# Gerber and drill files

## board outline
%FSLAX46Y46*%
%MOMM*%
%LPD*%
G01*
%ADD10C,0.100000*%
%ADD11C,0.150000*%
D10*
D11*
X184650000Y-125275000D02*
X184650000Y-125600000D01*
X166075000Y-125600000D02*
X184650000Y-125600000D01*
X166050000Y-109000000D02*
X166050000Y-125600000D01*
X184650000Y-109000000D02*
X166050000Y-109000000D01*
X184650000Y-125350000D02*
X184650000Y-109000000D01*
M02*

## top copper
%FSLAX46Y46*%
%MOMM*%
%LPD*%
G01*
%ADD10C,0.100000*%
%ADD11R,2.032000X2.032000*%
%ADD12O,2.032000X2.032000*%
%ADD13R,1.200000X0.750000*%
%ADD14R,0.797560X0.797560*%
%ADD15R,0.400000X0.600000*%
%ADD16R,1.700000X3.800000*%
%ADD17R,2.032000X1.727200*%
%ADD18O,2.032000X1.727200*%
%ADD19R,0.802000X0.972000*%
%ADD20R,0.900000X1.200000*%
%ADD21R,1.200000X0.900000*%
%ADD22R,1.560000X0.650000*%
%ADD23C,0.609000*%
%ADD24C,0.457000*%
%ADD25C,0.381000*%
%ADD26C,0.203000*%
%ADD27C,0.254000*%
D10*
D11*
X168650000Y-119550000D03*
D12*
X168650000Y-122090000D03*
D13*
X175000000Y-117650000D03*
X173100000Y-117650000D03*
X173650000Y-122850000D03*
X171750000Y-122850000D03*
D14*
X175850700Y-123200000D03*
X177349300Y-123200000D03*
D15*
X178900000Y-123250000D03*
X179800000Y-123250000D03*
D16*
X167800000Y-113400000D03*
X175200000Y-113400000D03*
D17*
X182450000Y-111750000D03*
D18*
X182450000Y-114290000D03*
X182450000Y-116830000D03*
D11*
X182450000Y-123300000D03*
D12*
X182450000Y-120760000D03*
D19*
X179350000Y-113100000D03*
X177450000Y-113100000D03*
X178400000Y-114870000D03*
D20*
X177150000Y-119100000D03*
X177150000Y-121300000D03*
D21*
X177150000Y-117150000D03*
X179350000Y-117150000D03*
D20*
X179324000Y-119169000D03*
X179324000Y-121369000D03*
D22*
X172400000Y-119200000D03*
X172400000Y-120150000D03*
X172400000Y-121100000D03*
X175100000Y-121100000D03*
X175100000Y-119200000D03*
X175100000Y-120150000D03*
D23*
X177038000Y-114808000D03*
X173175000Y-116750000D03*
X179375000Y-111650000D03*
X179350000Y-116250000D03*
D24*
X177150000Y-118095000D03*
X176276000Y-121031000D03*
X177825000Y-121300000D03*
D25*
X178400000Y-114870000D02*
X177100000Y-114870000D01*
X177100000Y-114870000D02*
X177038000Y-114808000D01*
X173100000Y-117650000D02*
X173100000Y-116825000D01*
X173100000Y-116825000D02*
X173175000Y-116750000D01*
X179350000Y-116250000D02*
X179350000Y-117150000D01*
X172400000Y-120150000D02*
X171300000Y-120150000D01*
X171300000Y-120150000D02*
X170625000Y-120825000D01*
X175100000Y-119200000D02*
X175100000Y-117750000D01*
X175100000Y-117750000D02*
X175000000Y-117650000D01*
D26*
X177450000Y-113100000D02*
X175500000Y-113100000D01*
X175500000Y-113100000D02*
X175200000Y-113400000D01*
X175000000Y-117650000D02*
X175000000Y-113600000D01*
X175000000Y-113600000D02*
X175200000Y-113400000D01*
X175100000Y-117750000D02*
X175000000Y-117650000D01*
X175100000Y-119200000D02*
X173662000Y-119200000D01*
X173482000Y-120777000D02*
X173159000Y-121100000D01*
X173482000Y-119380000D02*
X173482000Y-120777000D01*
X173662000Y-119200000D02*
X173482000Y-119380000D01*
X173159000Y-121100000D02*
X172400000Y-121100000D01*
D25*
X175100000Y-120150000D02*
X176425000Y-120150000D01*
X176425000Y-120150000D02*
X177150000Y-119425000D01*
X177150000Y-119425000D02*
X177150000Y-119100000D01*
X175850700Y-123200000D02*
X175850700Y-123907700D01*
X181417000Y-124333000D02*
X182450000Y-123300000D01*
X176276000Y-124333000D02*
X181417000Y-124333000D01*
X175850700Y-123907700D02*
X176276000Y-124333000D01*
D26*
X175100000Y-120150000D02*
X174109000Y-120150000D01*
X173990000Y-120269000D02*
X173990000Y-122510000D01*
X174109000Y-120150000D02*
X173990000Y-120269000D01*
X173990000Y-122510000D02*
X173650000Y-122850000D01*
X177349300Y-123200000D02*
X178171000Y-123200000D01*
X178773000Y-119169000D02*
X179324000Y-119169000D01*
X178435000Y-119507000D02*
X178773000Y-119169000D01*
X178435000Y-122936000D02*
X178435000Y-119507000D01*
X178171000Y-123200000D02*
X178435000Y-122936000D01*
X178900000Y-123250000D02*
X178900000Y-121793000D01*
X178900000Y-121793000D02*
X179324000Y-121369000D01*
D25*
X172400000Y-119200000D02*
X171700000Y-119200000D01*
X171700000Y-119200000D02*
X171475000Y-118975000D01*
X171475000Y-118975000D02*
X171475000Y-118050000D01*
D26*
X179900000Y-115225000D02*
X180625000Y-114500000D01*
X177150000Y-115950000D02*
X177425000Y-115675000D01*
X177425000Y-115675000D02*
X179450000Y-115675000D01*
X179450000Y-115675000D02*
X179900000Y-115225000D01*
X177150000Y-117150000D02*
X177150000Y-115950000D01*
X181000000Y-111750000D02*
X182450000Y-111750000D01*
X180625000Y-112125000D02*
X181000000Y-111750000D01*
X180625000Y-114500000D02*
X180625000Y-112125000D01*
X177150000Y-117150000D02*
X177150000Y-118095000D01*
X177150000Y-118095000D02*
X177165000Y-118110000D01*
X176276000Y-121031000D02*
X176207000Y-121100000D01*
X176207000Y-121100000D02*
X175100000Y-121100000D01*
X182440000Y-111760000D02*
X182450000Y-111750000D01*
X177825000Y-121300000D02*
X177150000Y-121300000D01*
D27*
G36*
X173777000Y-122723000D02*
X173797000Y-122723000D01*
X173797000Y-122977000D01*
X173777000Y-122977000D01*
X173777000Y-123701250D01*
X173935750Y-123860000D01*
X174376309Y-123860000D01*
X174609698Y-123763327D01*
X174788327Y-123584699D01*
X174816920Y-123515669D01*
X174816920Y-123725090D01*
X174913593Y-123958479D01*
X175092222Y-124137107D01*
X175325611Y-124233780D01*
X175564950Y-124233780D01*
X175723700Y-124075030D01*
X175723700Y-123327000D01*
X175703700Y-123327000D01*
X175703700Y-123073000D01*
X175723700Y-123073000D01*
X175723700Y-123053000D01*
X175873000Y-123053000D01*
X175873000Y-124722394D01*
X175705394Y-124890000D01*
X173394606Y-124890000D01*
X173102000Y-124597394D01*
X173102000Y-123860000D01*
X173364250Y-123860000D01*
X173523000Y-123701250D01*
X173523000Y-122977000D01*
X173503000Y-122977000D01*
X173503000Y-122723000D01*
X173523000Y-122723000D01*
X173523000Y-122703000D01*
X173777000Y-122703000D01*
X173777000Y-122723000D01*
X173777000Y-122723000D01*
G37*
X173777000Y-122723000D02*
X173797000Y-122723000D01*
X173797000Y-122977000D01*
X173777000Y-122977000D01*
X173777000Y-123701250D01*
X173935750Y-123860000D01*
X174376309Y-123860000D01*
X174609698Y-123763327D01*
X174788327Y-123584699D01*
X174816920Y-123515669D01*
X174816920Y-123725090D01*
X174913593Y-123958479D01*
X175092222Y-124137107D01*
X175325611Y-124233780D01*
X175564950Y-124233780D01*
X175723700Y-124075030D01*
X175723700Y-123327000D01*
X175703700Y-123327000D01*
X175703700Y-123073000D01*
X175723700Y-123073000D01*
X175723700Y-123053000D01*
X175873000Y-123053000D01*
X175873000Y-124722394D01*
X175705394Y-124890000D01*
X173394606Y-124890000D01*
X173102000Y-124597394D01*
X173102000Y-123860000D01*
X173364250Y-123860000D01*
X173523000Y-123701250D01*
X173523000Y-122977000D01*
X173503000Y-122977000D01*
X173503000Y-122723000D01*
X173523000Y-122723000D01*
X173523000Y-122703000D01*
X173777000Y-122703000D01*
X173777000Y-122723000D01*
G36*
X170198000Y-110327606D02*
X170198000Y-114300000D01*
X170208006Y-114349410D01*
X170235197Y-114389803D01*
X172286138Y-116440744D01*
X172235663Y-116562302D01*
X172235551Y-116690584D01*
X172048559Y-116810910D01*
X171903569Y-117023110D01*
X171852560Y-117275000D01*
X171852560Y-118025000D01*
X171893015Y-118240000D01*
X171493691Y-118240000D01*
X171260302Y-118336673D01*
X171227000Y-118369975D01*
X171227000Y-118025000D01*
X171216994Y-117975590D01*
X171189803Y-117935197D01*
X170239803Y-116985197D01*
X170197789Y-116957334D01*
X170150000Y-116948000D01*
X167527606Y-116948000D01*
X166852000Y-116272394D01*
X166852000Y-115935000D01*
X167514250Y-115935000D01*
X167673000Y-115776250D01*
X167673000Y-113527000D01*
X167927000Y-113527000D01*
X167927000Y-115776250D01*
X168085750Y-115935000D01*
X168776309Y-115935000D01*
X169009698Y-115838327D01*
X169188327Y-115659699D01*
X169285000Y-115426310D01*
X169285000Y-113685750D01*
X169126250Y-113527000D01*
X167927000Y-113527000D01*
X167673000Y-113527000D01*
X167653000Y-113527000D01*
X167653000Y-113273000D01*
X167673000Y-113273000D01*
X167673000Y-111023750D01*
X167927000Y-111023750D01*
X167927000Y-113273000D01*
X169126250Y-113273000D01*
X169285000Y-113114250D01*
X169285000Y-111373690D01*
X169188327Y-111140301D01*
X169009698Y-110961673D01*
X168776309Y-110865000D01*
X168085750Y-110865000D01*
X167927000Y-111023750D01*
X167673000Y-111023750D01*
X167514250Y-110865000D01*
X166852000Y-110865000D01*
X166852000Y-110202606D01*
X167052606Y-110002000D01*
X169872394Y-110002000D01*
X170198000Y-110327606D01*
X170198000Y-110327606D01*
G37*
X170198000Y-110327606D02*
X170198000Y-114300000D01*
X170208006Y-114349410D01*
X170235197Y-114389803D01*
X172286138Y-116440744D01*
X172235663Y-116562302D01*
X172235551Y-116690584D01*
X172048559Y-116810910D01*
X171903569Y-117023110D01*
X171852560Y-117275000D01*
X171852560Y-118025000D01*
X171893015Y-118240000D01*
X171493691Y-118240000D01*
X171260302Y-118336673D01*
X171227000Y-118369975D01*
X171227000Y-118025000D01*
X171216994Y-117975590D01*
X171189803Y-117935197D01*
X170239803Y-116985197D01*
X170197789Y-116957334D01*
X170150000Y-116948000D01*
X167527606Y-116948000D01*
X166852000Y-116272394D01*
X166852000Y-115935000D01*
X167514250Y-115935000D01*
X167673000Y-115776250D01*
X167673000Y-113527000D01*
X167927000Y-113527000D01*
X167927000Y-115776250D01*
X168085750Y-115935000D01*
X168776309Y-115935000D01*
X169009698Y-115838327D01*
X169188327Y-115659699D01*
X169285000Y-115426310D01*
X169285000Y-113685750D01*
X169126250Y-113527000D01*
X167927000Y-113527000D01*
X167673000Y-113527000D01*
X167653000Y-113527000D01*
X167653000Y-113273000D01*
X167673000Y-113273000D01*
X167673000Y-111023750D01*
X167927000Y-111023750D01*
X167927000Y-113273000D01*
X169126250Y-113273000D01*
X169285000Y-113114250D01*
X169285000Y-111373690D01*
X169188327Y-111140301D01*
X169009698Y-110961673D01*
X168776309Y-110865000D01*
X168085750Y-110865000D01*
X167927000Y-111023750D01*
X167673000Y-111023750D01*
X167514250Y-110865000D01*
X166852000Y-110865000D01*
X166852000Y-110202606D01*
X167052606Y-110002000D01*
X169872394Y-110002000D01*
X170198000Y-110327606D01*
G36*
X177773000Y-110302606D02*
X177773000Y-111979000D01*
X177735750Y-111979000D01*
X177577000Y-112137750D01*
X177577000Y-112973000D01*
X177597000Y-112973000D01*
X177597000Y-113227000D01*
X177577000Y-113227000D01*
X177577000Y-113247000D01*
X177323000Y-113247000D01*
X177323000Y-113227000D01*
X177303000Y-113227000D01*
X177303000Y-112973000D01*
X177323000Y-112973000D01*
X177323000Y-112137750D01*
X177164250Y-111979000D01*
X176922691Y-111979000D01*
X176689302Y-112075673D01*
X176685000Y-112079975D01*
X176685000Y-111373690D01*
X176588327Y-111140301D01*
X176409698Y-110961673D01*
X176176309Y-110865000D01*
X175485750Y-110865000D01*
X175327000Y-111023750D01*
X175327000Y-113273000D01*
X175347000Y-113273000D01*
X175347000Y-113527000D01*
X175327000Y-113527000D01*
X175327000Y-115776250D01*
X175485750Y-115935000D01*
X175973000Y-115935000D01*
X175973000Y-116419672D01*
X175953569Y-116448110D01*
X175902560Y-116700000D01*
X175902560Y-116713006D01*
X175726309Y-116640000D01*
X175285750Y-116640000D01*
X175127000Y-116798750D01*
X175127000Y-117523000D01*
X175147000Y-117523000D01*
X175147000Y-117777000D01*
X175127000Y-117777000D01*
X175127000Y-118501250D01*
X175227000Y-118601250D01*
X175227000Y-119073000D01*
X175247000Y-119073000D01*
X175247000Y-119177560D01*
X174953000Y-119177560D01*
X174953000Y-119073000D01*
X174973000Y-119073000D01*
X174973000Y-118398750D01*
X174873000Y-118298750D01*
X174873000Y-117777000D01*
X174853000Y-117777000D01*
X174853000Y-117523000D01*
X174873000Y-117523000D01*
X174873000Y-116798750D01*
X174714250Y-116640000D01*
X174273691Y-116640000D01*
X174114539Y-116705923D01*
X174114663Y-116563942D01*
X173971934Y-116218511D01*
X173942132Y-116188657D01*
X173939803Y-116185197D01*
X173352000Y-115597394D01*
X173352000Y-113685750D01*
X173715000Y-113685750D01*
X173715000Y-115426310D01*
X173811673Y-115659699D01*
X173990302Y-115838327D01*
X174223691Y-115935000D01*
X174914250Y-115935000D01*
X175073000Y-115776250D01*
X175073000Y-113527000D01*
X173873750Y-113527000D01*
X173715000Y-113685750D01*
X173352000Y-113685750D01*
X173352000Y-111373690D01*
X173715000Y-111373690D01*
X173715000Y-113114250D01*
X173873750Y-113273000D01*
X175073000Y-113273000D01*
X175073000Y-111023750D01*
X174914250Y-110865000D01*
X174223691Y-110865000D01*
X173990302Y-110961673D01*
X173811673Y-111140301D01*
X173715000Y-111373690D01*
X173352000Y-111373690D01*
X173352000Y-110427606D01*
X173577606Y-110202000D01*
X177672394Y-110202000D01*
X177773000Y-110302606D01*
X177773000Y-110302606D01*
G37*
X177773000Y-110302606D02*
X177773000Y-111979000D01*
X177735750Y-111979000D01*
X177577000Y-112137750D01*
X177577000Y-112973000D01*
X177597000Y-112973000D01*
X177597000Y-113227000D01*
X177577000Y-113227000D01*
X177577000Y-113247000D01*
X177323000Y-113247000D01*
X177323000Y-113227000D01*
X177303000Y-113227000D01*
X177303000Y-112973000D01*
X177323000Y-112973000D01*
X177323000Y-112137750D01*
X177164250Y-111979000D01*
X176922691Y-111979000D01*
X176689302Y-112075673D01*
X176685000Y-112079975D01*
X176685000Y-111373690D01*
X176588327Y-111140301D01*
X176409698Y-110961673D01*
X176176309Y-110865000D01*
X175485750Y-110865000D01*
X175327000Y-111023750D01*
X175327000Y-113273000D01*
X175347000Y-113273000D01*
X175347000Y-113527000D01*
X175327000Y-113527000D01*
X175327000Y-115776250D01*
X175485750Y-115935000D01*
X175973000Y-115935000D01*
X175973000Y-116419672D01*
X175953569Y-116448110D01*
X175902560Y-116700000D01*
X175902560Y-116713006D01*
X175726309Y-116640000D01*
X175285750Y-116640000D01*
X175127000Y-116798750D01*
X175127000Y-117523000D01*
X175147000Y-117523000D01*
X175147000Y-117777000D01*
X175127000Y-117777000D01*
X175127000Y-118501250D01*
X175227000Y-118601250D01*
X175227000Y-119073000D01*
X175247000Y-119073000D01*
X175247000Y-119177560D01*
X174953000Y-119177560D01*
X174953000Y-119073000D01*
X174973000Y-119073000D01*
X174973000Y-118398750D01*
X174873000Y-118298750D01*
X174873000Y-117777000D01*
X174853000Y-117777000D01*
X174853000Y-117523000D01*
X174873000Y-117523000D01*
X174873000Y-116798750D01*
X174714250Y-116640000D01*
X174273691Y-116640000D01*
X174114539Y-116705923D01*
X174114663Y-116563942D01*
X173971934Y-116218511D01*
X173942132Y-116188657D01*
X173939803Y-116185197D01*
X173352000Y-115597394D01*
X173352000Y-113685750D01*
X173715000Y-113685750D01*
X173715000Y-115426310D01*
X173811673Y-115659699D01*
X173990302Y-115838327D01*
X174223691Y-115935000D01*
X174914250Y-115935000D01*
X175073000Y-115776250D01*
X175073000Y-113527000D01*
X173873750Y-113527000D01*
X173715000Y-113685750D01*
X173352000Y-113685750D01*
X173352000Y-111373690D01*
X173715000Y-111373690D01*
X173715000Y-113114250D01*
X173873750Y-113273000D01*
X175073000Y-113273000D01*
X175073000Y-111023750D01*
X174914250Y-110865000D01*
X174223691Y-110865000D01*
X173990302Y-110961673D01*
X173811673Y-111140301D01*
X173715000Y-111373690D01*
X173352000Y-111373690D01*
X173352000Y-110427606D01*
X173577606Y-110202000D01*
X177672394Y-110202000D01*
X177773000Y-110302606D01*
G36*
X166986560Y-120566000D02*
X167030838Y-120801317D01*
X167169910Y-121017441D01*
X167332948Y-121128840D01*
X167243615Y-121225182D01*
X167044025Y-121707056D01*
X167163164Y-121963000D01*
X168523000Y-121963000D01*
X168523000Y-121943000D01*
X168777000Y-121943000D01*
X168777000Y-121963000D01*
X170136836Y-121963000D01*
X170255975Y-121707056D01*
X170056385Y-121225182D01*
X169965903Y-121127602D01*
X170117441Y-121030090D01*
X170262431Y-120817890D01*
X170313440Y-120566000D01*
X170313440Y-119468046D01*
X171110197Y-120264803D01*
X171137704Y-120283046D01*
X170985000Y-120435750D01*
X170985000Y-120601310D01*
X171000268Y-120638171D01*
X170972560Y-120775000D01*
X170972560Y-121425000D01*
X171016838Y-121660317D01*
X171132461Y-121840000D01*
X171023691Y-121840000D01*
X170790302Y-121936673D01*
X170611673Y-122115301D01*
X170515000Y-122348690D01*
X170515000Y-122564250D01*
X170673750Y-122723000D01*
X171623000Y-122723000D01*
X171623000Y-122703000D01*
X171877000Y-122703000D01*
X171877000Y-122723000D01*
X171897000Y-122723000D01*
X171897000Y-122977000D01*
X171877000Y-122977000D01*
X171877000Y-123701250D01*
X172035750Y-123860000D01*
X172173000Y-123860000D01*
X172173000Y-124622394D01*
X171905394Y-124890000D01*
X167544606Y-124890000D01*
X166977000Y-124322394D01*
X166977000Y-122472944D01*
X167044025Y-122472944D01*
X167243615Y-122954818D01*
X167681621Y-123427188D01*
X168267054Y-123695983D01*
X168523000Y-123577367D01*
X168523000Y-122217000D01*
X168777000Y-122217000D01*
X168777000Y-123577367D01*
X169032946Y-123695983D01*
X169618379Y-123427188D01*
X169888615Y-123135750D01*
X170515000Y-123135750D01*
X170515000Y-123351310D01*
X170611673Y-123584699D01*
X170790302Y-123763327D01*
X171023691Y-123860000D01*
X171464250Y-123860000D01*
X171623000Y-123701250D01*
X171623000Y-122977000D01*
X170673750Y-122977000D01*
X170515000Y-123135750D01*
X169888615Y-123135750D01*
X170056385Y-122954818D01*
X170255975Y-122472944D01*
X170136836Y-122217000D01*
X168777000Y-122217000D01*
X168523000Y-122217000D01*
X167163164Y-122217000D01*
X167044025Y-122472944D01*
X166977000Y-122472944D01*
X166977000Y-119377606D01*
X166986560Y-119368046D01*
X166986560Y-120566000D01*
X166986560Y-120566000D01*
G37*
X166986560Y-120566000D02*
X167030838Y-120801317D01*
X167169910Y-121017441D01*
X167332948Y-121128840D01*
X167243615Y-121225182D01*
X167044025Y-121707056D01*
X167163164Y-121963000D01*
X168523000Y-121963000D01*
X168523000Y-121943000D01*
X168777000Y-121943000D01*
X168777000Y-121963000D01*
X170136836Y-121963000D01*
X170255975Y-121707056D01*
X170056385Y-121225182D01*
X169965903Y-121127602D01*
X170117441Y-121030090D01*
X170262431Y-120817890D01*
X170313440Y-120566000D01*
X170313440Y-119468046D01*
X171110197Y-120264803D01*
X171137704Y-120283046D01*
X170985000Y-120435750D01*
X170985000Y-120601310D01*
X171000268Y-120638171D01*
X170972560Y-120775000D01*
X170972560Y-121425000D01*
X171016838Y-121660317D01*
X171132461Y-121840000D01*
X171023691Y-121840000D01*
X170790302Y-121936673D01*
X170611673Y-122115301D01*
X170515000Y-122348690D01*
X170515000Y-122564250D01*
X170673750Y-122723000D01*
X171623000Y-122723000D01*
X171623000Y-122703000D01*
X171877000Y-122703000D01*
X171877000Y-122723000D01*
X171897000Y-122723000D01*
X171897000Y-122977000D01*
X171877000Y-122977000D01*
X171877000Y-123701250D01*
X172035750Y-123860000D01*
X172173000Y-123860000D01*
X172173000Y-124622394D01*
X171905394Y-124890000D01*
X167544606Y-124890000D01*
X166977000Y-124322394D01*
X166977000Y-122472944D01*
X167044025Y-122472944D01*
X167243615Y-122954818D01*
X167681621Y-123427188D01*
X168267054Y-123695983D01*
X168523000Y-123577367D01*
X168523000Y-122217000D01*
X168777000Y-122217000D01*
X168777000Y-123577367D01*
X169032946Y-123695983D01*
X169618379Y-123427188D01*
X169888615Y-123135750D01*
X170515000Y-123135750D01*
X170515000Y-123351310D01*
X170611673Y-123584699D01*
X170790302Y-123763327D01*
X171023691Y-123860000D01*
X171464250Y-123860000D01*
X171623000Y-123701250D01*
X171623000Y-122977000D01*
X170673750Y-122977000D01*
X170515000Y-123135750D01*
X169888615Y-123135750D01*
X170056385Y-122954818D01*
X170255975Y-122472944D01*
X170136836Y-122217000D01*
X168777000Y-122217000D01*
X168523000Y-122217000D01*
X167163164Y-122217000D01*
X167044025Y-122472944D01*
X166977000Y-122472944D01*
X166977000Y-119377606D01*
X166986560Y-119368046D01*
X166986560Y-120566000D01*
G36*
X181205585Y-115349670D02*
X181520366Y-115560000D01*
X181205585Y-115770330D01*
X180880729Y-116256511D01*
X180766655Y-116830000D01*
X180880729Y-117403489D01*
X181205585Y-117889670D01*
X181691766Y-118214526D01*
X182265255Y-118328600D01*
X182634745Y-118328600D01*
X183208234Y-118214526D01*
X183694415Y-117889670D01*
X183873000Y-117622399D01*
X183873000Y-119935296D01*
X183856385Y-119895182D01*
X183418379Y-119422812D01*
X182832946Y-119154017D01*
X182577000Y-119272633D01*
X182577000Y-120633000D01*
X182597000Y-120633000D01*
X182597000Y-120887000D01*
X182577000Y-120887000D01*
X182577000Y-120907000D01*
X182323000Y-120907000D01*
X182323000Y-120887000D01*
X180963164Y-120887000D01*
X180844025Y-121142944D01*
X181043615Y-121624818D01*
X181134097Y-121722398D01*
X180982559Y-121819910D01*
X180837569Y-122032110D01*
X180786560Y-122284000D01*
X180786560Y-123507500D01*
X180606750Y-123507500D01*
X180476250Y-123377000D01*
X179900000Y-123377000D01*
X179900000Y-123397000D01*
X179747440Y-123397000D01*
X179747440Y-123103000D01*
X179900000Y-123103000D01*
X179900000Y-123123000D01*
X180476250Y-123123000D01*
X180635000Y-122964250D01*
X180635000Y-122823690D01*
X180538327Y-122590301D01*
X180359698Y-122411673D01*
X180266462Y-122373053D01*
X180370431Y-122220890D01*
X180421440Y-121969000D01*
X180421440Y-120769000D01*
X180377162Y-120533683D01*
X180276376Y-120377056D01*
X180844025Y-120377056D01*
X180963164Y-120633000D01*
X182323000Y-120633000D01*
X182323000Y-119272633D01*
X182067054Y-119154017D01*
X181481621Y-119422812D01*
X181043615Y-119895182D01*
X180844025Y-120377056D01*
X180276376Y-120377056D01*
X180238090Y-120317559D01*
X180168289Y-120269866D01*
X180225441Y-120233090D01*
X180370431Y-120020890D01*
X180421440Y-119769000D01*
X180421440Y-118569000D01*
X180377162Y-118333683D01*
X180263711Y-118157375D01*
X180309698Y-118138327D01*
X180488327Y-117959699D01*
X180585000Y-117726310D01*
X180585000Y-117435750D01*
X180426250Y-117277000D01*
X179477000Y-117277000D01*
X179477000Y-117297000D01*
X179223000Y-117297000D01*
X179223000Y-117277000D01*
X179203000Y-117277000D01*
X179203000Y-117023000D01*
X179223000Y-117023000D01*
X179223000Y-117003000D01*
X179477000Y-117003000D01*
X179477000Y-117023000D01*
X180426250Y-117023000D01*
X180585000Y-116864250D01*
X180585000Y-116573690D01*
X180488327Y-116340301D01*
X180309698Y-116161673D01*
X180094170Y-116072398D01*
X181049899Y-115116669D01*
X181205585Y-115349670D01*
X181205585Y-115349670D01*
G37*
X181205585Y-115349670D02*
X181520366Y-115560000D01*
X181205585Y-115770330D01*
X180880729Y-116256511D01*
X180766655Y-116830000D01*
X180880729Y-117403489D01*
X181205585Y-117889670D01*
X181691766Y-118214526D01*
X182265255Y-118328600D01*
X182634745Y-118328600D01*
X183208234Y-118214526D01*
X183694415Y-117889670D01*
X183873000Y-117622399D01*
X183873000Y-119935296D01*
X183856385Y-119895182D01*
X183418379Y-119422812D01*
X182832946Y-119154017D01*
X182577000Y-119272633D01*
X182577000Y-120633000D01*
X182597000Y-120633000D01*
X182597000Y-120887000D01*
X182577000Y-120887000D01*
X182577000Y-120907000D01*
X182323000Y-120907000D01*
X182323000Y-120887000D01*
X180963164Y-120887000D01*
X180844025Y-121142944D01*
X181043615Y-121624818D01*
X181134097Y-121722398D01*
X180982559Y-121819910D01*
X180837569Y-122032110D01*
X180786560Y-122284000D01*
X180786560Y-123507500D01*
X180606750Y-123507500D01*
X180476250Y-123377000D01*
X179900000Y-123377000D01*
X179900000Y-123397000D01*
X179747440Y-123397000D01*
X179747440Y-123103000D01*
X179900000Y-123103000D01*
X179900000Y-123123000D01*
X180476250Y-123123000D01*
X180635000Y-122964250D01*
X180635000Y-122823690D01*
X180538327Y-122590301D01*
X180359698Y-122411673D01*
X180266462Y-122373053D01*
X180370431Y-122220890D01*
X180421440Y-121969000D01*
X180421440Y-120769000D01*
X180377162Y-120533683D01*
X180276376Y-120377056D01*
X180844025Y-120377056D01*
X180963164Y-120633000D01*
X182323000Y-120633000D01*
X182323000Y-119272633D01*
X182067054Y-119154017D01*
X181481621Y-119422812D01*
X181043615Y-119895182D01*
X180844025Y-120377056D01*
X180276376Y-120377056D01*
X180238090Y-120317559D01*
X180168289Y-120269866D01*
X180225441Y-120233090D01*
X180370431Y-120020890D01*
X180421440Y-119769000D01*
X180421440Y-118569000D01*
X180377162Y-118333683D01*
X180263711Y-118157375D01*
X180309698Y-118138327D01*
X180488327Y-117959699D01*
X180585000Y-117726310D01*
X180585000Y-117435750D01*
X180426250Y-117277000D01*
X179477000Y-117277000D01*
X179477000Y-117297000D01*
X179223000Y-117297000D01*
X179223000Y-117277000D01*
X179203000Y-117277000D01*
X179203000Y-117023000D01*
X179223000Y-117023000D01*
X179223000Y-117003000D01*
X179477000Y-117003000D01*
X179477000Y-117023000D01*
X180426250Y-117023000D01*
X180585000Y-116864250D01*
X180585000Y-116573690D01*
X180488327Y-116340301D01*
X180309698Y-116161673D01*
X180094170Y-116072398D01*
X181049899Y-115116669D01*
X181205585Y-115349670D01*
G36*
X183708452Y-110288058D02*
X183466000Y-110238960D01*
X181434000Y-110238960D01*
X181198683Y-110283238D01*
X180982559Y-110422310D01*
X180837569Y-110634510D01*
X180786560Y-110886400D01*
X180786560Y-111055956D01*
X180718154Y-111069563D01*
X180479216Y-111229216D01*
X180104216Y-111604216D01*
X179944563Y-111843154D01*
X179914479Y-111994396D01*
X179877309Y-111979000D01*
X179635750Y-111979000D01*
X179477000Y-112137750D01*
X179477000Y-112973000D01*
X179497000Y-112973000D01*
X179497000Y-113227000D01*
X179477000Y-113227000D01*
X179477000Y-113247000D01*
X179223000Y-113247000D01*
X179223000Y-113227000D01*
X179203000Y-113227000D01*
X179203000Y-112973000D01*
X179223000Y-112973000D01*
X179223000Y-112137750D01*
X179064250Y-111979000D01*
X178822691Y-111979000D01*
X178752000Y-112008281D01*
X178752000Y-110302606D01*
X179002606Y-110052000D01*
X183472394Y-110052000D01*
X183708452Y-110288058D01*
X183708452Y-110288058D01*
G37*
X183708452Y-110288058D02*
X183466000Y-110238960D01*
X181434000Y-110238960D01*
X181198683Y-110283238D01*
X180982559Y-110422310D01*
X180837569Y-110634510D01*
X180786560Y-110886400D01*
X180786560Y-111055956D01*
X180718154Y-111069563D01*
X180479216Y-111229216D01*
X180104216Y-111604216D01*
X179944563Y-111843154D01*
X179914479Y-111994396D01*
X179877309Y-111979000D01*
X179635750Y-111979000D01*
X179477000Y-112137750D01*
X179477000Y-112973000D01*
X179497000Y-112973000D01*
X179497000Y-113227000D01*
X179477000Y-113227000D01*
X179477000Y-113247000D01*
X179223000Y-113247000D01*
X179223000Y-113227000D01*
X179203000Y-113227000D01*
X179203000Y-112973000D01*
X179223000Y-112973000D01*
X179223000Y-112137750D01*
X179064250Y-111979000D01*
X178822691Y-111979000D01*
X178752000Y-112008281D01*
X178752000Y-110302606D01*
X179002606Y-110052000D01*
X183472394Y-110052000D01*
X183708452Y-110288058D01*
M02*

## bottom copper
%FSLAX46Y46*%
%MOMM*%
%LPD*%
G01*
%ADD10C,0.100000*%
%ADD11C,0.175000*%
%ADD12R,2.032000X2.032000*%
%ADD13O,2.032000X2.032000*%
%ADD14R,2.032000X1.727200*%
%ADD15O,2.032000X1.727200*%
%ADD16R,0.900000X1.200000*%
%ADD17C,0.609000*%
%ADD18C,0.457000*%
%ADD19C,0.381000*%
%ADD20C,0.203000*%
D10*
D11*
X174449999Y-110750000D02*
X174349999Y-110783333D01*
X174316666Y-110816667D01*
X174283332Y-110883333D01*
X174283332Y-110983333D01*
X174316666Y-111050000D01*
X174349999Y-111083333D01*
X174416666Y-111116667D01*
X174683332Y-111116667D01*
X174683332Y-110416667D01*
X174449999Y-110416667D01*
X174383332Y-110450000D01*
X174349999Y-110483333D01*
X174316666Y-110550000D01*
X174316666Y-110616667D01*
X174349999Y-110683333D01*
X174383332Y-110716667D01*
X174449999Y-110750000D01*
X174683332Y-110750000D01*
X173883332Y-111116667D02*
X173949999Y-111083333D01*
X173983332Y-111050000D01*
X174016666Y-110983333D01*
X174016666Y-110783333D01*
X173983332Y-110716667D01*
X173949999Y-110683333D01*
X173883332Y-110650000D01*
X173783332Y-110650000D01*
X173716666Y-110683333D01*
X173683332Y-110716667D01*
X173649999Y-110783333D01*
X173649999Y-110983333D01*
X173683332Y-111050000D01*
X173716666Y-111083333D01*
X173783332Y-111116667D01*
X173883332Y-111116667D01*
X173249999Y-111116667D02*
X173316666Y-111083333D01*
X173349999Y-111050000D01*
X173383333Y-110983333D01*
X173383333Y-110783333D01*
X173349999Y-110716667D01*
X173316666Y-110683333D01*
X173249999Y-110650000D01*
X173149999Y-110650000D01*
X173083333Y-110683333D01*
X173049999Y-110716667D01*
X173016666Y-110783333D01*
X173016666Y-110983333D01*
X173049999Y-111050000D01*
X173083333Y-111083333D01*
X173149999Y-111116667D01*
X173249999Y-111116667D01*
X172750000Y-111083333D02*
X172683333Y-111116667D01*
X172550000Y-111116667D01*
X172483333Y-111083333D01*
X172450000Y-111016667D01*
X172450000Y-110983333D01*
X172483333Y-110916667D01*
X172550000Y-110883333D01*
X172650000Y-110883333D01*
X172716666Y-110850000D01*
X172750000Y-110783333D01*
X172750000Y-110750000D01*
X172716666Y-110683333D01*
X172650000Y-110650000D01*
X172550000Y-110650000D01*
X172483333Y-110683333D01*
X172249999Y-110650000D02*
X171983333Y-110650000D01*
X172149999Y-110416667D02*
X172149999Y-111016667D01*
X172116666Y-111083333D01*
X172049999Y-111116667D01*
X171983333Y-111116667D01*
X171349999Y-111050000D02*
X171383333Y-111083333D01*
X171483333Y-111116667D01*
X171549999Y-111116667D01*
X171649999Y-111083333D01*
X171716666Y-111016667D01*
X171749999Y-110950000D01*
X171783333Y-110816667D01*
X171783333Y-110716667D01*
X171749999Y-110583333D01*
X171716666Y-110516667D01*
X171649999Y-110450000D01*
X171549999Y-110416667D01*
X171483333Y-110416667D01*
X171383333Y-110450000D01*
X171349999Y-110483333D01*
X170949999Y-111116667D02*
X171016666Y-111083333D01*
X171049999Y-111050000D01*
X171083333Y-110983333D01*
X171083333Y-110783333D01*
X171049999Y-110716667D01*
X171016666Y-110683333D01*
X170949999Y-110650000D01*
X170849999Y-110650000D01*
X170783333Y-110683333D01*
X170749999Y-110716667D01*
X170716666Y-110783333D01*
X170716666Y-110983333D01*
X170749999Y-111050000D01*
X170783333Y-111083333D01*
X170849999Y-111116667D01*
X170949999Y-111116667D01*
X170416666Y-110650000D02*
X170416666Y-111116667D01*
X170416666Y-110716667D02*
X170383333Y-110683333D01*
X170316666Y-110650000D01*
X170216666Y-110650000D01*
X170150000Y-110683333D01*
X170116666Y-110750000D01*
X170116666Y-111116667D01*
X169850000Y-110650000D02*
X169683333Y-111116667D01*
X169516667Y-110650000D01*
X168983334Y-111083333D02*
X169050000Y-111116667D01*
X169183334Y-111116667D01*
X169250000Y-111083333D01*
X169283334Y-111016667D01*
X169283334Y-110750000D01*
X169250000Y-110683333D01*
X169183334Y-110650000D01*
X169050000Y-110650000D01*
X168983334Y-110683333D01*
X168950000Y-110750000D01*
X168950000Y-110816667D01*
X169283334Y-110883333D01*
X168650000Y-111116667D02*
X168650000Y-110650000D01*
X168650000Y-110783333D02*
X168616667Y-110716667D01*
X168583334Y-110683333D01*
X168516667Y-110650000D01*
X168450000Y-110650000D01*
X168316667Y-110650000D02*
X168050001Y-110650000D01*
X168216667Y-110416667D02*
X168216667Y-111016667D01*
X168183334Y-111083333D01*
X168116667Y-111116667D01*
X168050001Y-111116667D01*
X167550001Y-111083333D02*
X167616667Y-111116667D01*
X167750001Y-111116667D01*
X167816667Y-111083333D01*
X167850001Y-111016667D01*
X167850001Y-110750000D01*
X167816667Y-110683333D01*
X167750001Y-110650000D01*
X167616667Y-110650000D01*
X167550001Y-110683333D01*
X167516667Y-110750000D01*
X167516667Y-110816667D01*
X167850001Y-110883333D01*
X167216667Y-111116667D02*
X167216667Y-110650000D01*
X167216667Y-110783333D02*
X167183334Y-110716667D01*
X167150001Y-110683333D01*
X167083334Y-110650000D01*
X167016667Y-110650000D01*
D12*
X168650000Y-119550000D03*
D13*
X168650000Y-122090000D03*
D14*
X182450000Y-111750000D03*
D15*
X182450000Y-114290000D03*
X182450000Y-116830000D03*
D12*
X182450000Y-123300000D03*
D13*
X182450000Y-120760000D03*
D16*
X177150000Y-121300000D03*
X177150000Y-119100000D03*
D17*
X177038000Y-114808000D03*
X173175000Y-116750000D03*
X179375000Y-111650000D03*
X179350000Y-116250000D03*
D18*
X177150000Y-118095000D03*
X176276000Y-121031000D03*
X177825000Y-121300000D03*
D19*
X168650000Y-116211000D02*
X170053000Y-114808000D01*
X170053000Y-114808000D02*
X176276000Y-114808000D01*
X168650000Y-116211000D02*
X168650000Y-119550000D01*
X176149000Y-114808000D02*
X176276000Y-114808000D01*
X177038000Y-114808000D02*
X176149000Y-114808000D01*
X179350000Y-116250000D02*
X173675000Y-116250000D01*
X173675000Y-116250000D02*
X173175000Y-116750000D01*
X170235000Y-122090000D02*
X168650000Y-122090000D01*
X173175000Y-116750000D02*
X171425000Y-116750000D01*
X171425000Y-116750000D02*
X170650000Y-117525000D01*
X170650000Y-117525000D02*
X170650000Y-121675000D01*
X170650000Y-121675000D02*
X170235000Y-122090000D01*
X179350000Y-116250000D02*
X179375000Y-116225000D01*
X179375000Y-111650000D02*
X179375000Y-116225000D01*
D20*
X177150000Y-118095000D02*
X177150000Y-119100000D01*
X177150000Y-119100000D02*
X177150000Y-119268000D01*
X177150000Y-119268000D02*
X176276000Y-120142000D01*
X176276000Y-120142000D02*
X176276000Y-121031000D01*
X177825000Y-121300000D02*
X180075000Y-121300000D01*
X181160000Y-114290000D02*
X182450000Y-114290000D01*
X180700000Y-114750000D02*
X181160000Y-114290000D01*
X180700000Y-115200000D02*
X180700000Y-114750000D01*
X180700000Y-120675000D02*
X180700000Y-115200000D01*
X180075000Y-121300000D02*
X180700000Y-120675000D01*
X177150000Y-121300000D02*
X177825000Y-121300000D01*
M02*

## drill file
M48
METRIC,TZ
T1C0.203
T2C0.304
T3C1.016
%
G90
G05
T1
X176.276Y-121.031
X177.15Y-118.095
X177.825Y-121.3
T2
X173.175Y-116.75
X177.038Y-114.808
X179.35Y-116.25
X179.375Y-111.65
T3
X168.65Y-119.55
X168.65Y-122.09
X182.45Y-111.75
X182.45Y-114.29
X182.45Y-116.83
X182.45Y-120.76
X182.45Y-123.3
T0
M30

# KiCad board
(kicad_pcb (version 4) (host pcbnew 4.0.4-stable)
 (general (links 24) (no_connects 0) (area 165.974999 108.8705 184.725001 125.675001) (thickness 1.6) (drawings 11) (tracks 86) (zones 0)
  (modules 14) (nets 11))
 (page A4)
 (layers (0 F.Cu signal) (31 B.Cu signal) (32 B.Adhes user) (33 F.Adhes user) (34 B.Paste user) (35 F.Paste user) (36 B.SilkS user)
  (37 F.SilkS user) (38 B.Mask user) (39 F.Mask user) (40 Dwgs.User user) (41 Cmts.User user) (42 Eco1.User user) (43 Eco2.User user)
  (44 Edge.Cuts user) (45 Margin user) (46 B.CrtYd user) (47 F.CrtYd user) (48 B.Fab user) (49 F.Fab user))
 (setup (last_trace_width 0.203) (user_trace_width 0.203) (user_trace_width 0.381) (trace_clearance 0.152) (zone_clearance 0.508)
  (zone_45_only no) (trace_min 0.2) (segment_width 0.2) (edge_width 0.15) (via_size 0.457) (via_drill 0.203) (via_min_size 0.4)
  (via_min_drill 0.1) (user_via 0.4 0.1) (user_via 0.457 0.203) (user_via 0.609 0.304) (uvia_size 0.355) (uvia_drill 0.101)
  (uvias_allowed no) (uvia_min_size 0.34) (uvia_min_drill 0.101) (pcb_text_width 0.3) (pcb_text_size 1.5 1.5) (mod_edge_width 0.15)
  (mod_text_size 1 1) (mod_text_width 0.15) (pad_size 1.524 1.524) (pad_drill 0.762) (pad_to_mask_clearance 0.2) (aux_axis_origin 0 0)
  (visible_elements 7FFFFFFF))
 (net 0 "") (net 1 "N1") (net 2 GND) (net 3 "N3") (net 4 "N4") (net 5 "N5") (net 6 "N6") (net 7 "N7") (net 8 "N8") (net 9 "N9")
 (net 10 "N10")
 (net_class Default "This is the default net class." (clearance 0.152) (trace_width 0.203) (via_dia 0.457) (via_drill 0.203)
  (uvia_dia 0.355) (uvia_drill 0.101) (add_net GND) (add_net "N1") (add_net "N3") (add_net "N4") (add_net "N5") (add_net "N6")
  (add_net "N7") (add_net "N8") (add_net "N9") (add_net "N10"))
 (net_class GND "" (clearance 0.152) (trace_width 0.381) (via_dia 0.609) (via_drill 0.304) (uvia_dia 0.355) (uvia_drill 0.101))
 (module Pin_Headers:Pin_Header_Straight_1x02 (layer F.Cu) (at 168.65 119.55)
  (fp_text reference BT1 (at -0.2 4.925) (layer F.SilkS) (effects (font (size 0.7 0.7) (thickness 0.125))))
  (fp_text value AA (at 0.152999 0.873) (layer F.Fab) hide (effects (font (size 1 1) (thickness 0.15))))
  (pad 1 thru_hole rect (at 0 0) (size 2.032 2.032) (drill 1.016) (layers *.Cu *.Mask F.SilkS) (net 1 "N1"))
  (pad 2 thru_hole oval (at 0 2.54) (size 2.032 2.032) (drill 1.016) (layers *.Cu *.Mask F.SilkS) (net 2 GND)))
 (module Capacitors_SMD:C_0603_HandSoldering (layer F.Cu) (at 174.05 117.65 180)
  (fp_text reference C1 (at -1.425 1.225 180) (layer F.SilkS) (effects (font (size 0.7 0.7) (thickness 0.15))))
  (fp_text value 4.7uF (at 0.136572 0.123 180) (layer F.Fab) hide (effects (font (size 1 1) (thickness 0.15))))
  (pad 1 smd rect (at -0.95 0 180) (size 1.2 0.75) (layers F.Cu F.Paste F.Mask) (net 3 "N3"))
  (pad 2 smd rect (at 0.95 0 180) (size 1.2 0.75) (layers F.Cu F.Paste F.Mask) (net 2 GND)))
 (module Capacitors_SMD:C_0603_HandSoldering (layer F.Cu) (at 172.7 122.85 180)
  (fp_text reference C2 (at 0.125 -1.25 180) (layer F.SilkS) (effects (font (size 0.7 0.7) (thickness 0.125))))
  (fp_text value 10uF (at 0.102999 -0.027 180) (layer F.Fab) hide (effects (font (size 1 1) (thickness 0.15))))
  (pad 1 smd rect (at -0.95 0 180) (size 1.2 0.75) (layers F.Cu F.Paste F.Mask) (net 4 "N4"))
  (pad 2 smd rect (at 0.95 0 180) (size 1.2 0.75) (layers F.Cu F.Paste F.Mask) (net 2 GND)))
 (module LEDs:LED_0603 (layer F.Cu) (at 176.6 123.2 180)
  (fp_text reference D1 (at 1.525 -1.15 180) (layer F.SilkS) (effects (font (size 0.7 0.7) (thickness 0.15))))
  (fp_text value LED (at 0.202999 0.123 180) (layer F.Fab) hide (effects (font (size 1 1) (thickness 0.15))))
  (pad 2 smd rect (at 0.7493 0) (size 0.79756 0.79756) (layers F.Cu F.Paste F.Mask) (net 4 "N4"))
  (pad 1 smd rect (at -0.7493 0) (size 0.79756 0.79756) (layers F.Cu F.Paste F.Mask) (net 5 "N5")))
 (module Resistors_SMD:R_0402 (layer F.Cu) (at 179.35 123.25)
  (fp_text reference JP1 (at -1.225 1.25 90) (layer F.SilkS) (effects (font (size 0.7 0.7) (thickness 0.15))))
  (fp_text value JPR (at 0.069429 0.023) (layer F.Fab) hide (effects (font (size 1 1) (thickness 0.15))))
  (pad 1 smd rect (at -0.45 0) (size 0.4 0.6) (layers F.Cu F.Paste F.Mask) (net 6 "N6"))
  (pad 2 smd rect (at 0.45 0) (size 0.4 0.6) (layers F.Cu F.Paste F.Mask) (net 2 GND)))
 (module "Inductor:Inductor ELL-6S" (layer F.Cu) (at 171.5 113.4 180)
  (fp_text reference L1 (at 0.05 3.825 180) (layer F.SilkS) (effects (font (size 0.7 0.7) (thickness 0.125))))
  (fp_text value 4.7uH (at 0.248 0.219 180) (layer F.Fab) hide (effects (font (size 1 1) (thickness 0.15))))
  (pad 2 smd rect (at 3.7 0 180) (size 1.7 3.8) (layers F.Cu F.Paste F.Mask) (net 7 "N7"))
  (pad 1 smd rect (at -3.7 0 180) (size 1.7 3.8) (layers F.Cu F.Paste F.Mask) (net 3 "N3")))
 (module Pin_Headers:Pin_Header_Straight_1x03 (layer F.Cu) (at 182.45 111.75)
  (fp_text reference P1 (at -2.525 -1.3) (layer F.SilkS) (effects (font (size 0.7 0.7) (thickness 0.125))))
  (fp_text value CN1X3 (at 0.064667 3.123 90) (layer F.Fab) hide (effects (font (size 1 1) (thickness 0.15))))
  (pad 1 thru_hole rect (at 0 0) (size 2.032 1.7272) (drill 1.016) (layers *.Cu *.Mask F.SilkS) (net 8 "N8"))
  (pad 2 thru_hole oval (at 0 2.54) (size 2.032 1.7272) (drill 1.016) (layers *.Cu *.Mask F.SilkS) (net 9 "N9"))
  (pad 3 thru_hole oval (at 0 5.08) (size 2.032 1.7272) (drill 1.016) (layers *.Cu *.Mask F.SilkS) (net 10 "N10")))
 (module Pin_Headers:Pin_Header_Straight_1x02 (layer F.Cu) (at 182.45 123.3 180)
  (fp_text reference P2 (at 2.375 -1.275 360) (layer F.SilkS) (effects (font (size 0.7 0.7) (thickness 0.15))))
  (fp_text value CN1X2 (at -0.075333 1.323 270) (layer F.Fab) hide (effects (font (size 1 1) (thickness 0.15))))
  (pad 1 thru_hole rect (at 0 0 180) (size 2.032 2.032) (drill 1.016) (layers *.Cu *.Mask F.SilkS) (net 4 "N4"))
  (pad 2 thru_hole oval (at 0 2.54 180) (size 2.032 2.032) (drill 1.016) (layers *.Cu *.Mask F.SilkS) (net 2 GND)))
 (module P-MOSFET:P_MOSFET (layer F.Cu) (at 178.4 113.1 180)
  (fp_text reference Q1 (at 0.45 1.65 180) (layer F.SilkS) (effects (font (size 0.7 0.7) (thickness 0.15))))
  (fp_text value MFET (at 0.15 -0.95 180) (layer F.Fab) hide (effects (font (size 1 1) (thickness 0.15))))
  (pad 1 smd rect (at -0.95 0 180) (size 0.802 0.972) (layers F.Cu F.Paste F.Mask) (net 2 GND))
  (pad 2 smd rect (at 0.95 0 180) (size 0.802 0.972) (layers F.Cu F.Paste F.Mask) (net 3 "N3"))
  (pad 3 smd rect (at 0 -1.77 180) (size 0.802 0.972) (layers F.Cu F.Paste F.Mask) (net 1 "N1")))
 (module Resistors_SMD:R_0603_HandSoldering (layer F.Cu) (at 177.15 120.2 270)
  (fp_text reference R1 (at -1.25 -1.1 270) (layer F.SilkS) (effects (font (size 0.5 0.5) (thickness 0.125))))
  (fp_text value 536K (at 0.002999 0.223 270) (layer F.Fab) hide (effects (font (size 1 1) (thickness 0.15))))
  (pad 1 smd rect (at -1.1 0 270) (size 1.2 0.9) (layers F.Cu F.Paste F.Mask) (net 4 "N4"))
  (pad 2 smd rect (at 1.1 0 270) (size 1.2 0.9) (layers F.Cu F.Paste F.Mask) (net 9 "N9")))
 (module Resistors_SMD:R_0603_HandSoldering (layer B.Cu) (at 177.15 120.2 90)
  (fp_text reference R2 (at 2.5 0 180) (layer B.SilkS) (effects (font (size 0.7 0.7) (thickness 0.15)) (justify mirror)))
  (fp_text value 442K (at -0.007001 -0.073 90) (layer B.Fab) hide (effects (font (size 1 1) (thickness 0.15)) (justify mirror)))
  (pad 1 smd rect (at -1.1 0 90) (size 1.2 0.9) (layers B.Cu B.Paste B.Mask) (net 9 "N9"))
  (pad 2 smd rect (at 1.1 0 90) (size 1.2 0.9) (layers B.Cu B.Paste B.Mask) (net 8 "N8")))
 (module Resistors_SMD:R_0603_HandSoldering (layer F.Cu) (at 178.25 117.15)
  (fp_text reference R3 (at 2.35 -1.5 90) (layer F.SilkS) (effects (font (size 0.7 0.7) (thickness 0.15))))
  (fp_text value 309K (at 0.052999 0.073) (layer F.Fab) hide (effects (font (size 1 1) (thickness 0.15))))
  (pad 1 smd rect (at -1.1 0) (size 1.2 0.9) (layers F.Cu F.Paste F.Mask) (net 8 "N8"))
  (pad 2 smd rect (at 1.1 0) (size 1.2 0.9) (layers F.Cu F.Paste F.Mask) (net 2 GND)))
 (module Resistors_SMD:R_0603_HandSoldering (layer F.Cu) (at 179.324 120.269 270)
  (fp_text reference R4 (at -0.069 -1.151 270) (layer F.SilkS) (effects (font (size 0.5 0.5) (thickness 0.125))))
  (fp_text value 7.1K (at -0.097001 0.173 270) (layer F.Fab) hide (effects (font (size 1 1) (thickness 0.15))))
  (pad 1 smd rect (at -1.1 0 270) (size 1.2 0.9) (layers F.Cu F.Paste F.Mask) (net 5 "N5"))
  (pad 2 smd rect (at 1.1 0 270) (size 1.2 0.9) (layers F.Cu F.Paste F.Mask) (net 6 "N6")))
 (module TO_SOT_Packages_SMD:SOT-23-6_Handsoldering (layer F.Cu) (at 173.75 120.15)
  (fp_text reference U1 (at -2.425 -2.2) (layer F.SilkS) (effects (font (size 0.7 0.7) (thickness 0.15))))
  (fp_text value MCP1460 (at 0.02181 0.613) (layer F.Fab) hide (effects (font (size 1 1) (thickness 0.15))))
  (pad 1 smd rect (at -1.35 -0.95) (size 1.56 0.65) (layers F.Cu F.Paste F.Mask) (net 7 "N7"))
  (pad 2 smd rect (at -1.35 0) (size 1.56 0.65) (layers F.Cu F.Paste F.Mask) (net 2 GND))
  (pad 3 smd rect (at -1.35 0.95) (size 1.56 0.65) (layers F.Cu F.Paste F.Mask) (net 3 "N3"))
  (pad 4 smd rect (at 1.35 0.95) (size 1.56 0.65) (layers F.Cu F.Paste F.Mask) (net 8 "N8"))
  (pad 6 smd rect (at 1.35 -0.95) (size 1.56 0.65) (layers F.Cu F.Paste F.Mask) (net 3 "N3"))
  (pad 5 smd rect (at 1.35 0) (size 1.56 0.65) (layers F.Cu F.Paste F.Mask) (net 4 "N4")))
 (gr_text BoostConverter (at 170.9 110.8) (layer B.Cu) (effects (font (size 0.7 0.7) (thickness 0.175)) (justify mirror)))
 (gr_line (start 184.65 125.275) (end 184.65 125.6) (angle 90) (layer Edge.Cuts) (width 0.15))
 (gr_line (start 166.075 125.6) (end 184.65 125.6) (angle 90) (layer Edge.Cuts) (width 0.15))
 (gr_line (start 166.05 109) (end 166.05 125.6) (angle 90) (layer Edge.Cuts) (width 0.15))
 (gr_line (start 184.65 109) (end 166.05 109) (angle 90) (layer Edge.Cuts) (width 0.15))
 (gr_line (start 184.65 125.35) (end 184.65 109) (angle 90) (layer Edge.Cuts) (width 0.15))
 (segment (start 178.4 114.87) (end 177.1 114.87) (width 0.381) (layer F.Cu) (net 1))
 (segment (start 168.65 116.211) (end 170.053 114.808) (width 0.381) (layer B.Cu) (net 1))
 (segment (start 170.053 114.808) (end 176.276 114.808) (width 0.381) (layer B.Cu) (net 1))
 (segment (start 168.65 116.211) (end 168.65 119.55) (width 0.381) (layer B.Cu) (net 1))
 (segment (start 176.149 114.808) (end 176.276 114.808) (width 0.381) (layer B.Cu) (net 1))
 (segment (start 177.038 114.808) (end 176.149 114.808) (width 0.381) (layer B.Cu) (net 1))
 (via (at 177.038 114.808) (size 0.609) (drill 0.304) (layers F.Cu B.Cu) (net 1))
 (segment (start 177.1 114.87) (end 177.038 114.808) (width 0.381) (layer F.Cu) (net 1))
 (segment (start 179.35 116.25) (end 173.675 116.25) (width 0.381) (layer B.Cu) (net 2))
 (segment (start 173.675 116.25) (end 173.175 116.75) (width 0.381) (layer B.Cu) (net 2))
 (segment (start 173.1 117.65) (end 173.1 116.825) (width 0.381) (layer F.Cu) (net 2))
 (segment (start 173.1 116.825) (end 173.175 116.75) (width 0.381) (layer F.Cu) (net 2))
 (via (at 173.175 116.75) (size 0.609) (drill 0.304) (layers F.Cu B.Cu) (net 2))
 (segment (start 170.235 122.09) (end 168.65 122.09) (width 0.381) (layer B.Cu) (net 2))
 (segment (start 173.175 116.75) (end 171.425 116.75) (width 0.381) (layer B.Cu) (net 2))
 (segment (start 171.425 116.75) (end 170.65 117.525) (width 0.381) (layer B.Cu) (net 2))
 (segment (start 170.65 117.525) (end 170.65 121.675) (width 0.381) (layer B.Cu) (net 2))
 (segment (start 170.65 121.675) (end 170.235 122.09) (width 0.381) (layer B.Cu) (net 2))
 (via (at 179.375 111.65) (size 0.609) (drill 0.304) (layers F.Cu B.Cu) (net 2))
 (via (at 179.35 116.25) (size 0.609) (drill 0.304) (layers F.Cu B.Cu) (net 2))
 (segment (start 179.35 116.25) (end 179.375 116.225) (width 0.381) (layer B.Cu) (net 2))
 (segment (start 179.375 111.65) (end 179.375 116.225) (width 0.381) (layer B.Cu) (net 2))
 (segment (start 179.35 116.25) (end 179.35 117.15) (width 0.381) (layer F.Cu) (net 2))
 (segment (start 172.4 120.15) (end 171.3 120.15) (width 0.381) (layer F.Cu) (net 2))
 (segment (start 171.3 120.15) (end 170.625 120.825) (width 0.381) (layer F.Cu) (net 2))
 (segment (start 175.1 119.2) (end 175.1 117.75) (width 0.381) (layer F.Cu) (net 3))
 (segment (start 175.1 117.75) (end 175 117.65) (width 0.381) (layer F.Cu) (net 3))
 (segment (start 177.45 113.1) (end 175.5 113.1) (width 0.203) (layer F.Cu) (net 3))
 (segment (start 175.5 113.1) (end 175.2 113.4) (width 0.203) (layer F.Cu) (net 3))
 (segment (start 175 117.65) (end 175 113.6) (width 0.203) (layer F.Cu) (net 3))
 (segment (start 175 113.6) (end 175.2 113.4) (width 0.203) (layer F.Cu) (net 3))
 (segment (start 175.1 117.75) (end 175 117.65) (width 0.203) (layer F.Cu) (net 3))
 (segment (start 175.1 119.2) (end 173.662 119.2) (width 0.203) (layer F.Cu) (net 3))
 (segment (start 173.482 120.777) (end 173.159 121.1) (width 0.203) (layer F.Cu) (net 3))
 (segment (start 173.482 119.38) (end 173.482 120.777) (width 0.203) (layer F.Cu) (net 3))
 (segment (start 173.662 119.2) (end 173.482 119.38) (width 0.203) (layer F.Cu) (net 3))
 (segment (start 173.159 121.1) (end 172.4 121.1) (width 0.203) (layer F.Cu) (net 3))
 (segment (start 175.1 120.15) (end 176.425 120.15) (width 0.381) (layer F.Cu) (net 4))
 (segment (start 176.425 120.15) (end 177.15 119.425) (width 0.381) (layer F.Cu) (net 4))
 (segment (start 177.15 119.425) (end 177.15 119.1) (width 0.381) (layer F.Cu) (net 4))
 (segment (start 175.8507 123.2) (end 175.8507 123.9077) (width 0.381) (layer F.Cu) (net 4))
 (segment (start 181.417 124.333) (end 182.45 123.3) (width 0.381) (layer F.Cu) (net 4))
 (segment (start 176.276 124.333) (end 181.417 124.333) (width 0.381) (layer F.Cu) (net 4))
 (segment (start 175.8507 123.9077) (end 176.276 124.333) (width 0.381) (layer F.Cu) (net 4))
 (segment (start 175.1 120.15) (end 174.109 120.15) (width 0.203) (layer F.Cu) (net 4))
 (segment (start 173.99 120.269) (end 173.99 122.51) (width 0.203) (layer F.Cu) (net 4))
 (segment (start 174.109 120.15) (end 173.99 120.269) (width 0.203) (layer F.Cu) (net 4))
 (segment (start 173.99 122.51) (end 173.65 122.85) (width 0.203) (layer F.Cu) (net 4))
 (segment (start 177.3493 123.2) (end 178.171 123.2) (width 0.203) (layer F.Cu) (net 5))
 (segment (start 178.773 119.169) (end 179.324 119.169) (width 0.203) (layer F.Cu) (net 5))
 (segment (start 178.435 119.507) (end 178.773 119.169) (width 0.203) (layer F.Cu) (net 5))
 (segment (start 178.435 122.936) (end 178.435 119.507) (width 0.203) (layer F.Cu) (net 5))
 (segment (start 178.171 123.2) (end 178.435 122.936) (width 0.203) (layer F.Cu) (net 5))
 (segment (start 178.9 123.25) (end 178.9 121.793) (width 0.203) (layer F.Cu) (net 6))
 (segment (start 178.9 121.793) (end 179.324 121.369) (width 0.203) (layer F.Cu) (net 6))
 (segment (start 172.4 119.2) (end 171.7 119.2) (width 0.381) (layer F.Cu) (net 7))
 (segment (start 171.7 119.2) (end 171.475 118.975) (width 0.381) (layer F.Cu) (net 7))
 (segment (start 171.475 118.975) (end 171.475 118.05) (width 0.381) (layer F.Cu) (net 7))
 (segment (start 179.9 115.225) (end 180.625 114.5) (width 0.203) (layer F.Cu) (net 8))
 (segment (start 177.15 115.95) (end 177.425 115.675) (width 0.203) (layer F.Cu) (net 8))
 (segment (start 177.425 115.675) (end 179.45 115.675) (width 0.203) (layer F.Cu) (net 8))
 (segment (start 179.45 115.675) (end 179.9 115.225) (width 0.203) (layer F.Cu) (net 8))
 (segment (start 177.15 117.15) (end 177.15 115.95) (width 0.203) (layer F.Cu) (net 8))
 (segment (start 181 111.75) (end 182.45 111.75) (width 0.203) (layer F.Cu) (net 8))
 (segment (start 180.625 112.125) (end 181 111.75) (width 0.203) (layer F.Cu) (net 8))
 (segment (start 180.625 114.5) (end 180.625 112.125) (width 0.203) (layer F.Cu) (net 8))
 (via (at 177.15 118.095) (size 0.457) (drill 0.203) (layers F.Cu B.Cu) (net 8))
 (segment (start 177.15 118.095) (end 177.15 119.1) (width 0.203) (layer B.Cu) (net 8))
 (segment (start 177.15 117.15) (end 177.15 118.095) (width 0.203) (layer F.Cu) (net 8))
 (segment (start 177.15 118.095) (end 177.165 118.11) (width 0.203) (layer F.Cu) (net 8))
 (segment (start 177.15 119.1) (end 177.15 119.268) (width 0.203) (layer B.Cu) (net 8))
 (segment (start 177.15 119.268) (end 176.276 120.142) (width 0.203) (layer B.Cu) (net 8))
 (segment (start 176.276 120.142) (end 176.276 121.031) (width 0.203) (layer B.Cu) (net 8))
 (via (at 176.276 121.031) (size 0.457) (drill 0.203) (layers F.Cu B.Cu) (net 8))
 (segment (start 176.276 121.031) (end 176.207 121.1) (width 0.203) (layer F.Cu) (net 8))
 (segment (start 176.207 121.1) (end 175.1 121.1) (width 0.203) (layer F.Cu) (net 8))
 (segment (start 182.44 111.76) (end 182.45 111.75) (width 0.203) (layer F.Cu) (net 8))
 (segment (start 177.825 121.3) (end 180.075 121.3) (width 0.203) (layer B.Cu) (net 9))
 (segment (start 181.16 114.29) (end 182.45 114.29) (width 0.203) (layer B.Cu) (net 9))
 (segment (start 180.7 114.75) (end 181.16 114.29) (width 0.203) (layer B.Cu) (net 9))
 (segment (start 180.7 115.2) (end 180.7 114.75) (width 0.203) (layer B.Cu) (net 9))
 (segment (start 180.7 120.675) (end 180.7 115.2) (width 0.203) (layer B.Cu) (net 9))
 (segment (start 180.075 121.3) (end 180.7 120.675) (width 0.203) (layer B.Cu) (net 9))
 (segment (start 177.15 121.3) (end 177.825 121.3) (width 0.203) (layer B.Cu) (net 9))
 (segment (start 177.825 121.3) (end 177.15 121.3) (width 0.203) (layer F.Cu) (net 9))
 (via (at 177.825 121.3) (size 0.457) (drill 0.203) (layers F.Cu B.Cu) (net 9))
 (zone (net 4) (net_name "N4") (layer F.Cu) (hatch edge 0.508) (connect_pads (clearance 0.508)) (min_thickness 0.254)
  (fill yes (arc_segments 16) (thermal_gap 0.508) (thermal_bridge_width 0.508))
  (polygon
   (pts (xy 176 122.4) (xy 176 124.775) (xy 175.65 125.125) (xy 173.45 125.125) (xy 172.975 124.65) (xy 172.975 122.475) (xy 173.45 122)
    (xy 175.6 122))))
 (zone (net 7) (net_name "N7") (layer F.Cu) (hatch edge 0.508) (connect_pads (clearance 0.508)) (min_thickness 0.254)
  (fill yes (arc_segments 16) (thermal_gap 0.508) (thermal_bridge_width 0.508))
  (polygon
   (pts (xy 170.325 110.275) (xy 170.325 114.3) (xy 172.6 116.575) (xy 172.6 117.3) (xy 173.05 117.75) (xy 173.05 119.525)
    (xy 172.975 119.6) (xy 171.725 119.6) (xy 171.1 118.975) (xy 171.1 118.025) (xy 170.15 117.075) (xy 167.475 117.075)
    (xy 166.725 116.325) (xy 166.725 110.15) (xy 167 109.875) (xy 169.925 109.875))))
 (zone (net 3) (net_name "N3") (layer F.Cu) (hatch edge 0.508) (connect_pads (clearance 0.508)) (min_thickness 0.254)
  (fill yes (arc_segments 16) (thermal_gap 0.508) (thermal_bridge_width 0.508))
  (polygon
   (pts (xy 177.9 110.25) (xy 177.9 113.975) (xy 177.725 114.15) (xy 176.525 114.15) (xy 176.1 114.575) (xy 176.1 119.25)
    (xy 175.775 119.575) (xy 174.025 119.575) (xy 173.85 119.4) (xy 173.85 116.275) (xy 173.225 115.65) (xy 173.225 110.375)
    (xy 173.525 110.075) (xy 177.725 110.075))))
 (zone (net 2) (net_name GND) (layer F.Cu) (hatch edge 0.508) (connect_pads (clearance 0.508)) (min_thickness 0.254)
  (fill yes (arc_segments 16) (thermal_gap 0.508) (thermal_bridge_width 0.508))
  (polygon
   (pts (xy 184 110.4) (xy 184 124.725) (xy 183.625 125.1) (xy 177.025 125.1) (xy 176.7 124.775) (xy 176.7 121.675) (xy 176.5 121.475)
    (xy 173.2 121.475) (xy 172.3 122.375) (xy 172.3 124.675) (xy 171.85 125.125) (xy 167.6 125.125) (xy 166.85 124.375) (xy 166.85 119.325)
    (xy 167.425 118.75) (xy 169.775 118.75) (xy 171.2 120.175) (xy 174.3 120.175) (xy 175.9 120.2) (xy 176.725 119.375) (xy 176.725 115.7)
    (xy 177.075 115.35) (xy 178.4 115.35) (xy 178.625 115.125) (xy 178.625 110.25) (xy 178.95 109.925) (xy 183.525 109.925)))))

